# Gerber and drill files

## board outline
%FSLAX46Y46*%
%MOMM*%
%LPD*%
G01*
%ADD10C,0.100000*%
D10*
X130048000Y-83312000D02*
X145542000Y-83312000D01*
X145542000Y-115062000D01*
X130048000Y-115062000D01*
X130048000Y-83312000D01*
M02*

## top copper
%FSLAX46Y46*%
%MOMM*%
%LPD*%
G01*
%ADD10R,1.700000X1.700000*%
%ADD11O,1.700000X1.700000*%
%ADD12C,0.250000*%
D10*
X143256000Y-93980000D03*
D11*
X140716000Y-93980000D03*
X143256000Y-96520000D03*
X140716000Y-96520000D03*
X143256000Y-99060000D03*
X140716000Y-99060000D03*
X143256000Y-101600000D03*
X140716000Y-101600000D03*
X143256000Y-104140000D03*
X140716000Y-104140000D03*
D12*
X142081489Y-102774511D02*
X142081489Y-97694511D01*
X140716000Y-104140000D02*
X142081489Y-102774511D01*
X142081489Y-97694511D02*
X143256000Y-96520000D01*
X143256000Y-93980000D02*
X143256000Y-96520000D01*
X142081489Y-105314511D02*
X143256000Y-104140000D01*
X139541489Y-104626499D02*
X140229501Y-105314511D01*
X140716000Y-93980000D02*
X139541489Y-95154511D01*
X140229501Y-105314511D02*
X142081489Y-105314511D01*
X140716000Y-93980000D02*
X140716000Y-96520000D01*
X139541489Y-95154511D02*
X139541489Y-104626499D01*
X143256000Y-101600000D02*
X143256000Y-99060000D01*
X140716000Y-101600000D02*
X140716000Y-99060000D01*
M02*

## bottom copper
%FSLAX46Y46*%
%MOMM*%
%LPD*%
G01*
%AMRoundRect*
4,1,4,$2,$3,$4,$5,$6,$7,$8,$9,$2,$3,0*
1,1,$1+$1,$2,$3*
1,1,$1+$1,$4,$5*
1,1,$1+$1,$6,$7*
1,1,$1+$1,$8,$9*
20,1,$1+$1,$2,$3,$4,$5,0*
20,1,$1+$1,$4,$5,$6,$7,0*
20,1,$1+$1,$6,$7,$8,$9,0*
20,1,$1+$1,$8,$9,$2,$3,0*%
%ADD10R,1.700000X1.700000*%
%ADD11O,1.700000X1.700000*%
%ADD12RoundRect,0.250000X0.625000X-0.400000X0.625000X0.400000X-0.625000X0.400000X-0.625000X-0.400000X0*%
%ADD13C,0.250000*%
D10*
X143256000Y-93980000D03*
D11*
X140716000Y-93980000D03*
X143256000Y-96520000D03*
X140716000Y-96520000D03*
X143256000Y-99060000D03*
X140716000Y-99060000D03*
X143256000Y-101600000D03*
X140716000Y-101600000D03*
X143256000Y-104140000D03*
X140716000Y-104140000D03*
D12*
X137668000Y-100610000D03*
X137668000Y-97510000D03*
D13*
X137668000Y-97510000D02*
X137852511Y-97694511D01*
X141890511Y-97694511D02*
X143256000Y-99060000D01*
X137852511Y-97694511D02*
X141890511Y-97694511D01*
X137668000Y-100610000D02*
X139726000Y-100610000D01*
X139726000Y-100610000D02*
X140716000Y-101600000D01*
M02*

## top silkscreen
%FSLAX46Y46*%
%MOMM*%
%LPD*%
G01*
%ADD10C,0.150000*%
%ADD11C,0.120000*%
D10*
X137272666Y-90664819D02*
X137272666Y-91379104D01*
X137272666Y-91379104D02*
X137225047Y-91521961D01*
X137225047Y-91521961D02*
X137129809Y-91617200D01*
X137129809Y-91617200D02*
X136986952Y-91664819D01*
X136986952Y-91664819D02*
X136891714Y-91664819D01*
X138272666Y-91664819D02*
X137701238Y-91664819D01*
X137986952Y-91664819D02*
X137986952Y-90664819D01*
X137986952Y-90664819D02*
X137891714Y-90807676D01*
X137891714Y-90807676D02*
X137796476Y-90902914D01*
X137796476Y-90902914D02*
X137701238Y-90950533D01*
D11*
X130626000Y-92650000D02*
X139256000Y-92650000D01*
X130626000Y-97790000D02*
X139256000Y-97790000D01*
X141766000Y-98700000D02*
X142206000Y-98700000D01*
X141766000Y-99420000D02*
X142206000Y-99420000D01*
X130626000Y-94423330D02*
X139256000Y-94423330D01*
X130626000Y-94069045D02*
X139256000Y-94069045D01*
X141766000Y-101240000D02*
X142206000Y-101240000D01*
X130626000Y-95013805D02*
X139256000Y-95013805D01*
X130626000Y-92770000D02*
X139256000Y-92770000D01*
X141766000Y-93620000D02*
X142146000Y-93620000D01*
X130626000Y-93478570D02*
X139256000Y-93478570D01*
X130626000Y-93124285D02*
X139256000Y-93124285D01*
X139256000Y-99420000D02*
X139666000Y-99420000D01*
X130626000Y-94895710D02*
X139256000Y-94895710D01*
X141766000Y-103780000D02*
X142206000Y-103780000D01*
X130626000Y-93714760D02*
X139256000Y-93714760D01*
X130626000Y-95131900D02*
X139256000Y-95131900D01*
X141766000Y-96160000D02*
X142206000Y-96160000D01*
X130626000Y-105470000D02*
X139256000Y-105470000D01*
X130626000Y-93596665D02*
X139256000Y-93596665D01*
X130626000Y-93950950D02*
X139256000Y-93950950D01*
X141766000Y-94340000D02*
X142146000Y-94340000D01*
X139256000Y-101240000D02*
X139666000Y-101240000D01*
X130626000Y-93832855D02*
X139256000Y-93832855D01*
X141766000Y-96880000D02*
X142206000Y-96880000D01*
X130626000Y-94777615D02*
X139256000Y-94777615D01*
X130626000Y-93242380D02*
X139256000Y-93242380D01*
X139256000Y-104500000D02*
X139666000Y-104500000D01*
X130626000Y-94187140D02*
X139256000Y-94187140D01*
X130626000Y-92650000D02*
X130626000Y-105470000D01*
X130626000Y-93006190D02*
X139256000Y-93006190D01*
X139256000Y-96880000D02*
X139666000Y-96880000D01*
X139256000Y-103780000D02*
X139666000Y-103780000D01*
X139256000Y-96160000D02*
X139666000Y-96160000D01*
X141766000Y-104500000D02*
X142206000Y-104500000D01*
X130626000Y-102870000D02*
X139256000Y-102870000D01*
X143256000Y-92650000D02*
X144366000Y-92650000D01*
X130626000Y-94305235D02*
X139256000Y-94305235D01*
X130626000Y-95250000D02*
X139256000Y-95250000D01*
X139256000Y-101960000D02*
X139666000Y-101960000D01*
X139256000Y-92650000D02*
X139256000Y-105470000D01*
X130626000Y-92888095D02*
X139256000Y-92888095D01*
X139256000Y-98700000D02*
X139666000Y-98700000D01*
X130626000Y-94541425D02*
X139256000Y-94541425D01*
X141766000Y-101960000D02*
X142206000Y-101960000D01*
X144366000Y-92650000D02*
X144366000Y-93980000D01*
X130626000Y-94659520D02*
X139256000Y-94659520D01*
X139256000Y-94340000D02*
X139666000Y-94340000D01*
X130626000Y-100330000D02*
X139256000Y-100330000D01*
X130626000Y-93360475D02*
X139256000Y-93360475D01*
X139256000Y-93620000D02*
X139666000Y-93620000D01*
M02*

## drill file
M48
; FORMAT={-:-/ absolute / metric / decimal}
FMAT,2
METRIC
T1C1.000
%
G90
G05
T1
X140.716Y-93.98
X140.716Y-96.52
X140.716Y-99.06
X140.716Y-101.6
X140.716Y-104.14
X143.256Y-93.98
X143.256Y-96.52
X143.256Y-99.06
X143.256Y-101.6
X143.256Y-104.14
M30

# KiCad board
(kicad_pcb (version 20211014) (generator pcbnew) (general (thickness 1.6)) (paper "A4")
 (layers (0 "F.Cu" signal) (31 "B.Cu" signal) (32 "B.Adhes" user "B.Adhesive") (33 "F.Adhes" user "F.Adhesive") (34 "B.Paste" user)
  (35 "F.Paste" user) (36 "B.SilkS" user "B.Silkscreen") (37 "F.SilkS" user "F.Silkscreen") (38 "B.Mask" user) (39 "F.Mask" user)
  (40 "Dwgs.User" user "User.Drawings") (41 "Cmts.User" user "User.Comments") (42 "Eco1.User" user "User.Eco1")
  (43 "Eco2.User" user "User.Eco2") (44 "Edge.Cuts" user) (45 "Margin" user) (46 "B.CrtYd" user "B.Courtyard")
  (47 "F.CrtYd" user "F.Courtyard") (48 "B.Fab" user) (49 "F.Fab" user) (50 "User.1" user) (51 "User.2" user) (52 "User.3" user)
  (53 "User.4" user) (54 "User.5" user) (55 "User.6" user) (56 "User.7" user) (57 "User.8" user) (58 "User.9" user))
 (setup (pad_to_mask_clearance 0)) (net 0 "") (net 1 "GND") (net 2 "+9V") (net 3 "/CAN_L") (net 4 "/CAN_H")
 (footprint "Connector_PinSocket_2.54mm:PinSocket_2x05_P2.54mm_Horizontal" (layer "F.Cu") (at 143.256 93.98)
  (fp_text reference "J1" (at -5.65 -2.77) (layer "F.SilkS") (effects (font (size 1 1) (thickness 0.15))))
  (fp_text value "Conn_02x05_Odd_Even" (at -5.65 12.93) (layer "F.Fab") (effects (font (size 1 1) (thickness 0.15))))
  (fp_line (start -12.63 -1.33) (end -4 -1.33) (layer "F.SilkS") (width 0.12))
  (fp_line (start -12.63 3.81) (end -4 3.81) (layer "F.SilkS") (width 0.12))
  (fp_line (start -1.49 4.72) (end -1.05 4.72) (layer "F.SilkS") (width 0.12))
  (fp_line (start -1.49 5.44) (end -1.05 5.44) (layer "F.SilkS") (width 0.12))
  (fp_line (start -12.63 0.44333) (end -4 0.44333) (layer "F.SilkS") (width 0.12))
  (fp_line (start -12.63 0.089045) (end -4 0.089045) (layer "F.SilkS") (width 0.12))
  (fp_line (start -1.49 7.26) (end -1.05 7.26) (layer "F.SilkS") (width 0.12))
  (fp_line (start -12.63 1.033805) (end -4 1.033805) (layer "F.SilkS") (width 0.12))
  (fp_line (start -12.63 -1.21) (end -4 -1.21) (layer "F.SilkS") (width 0.12))
  (fp_line (start -1.49 -0.36) (end -1.11 -0.36) (layer "F.SilkS") (width 0.12))
  (fp_line (start -12.63 -0.50143) (end -4 -0.50143) (layer "F.SilkS") (width 0.12))
  (fp_line (start -12.63 -0.855715) (end -4 -0.855715) (layer "F.SilkS") (width 0.12))
  (fp_line (start -4 5.44) (end -3.59 5.44) (layer "F.SilkS") (width 0.12))
  (fp_line (start -12.63 0.91571) (end -4 0.91571) (layer "F.SilkS") (width 0.12))
  (fp_line (start -1.49 9.8) (end -1.05 9.8) (layer "F.SilkS") (width 0.12))
  (fp_line (start -12.63 -0.26524) (end -4 -0.26524) (layer "F.SilkS") (width 0.12))
  (fp_line (start -12.63 1.1519) (end -4 1.1519) (layer "F.SilkS") (width 0.12))
  (fp_line (start -1.49 2.18) (end -1.05 2.18) (layer "F.SilkS") (width 0.12))
  (fp_line (start -12.63 11.49) (end -4 11.49) (layer "F.SilkS") (width 0.12))
  (fp_line (start -12.63 -0.383335) (end -4 -0.383335) (layer "F.SilkS") (width 0.12))
  (fp_line (start -12.63 -0.02905) (end -4 -0.02905) (layer "F.SilkS") (width 0.12))
  (fp_line (start -1.49 0.36) (end -1.11 0.36) (layer "F.SilkS") (width 0.12))
  (fp_line (start -4 7.26) (end -3.59 7.26) (layer "F.SilkS") (width 0.12))
  (fp_line (start -12.63 -0.147145) (end -4 -0.147145) (layer "F.SilkS") (width 0.12))
  (fp_line (start -1.49 2.9) (end -1.05 2.9) (layer "F.SilkS") (width 0.12))
  (fp_line (start -12.63 0.797615) (end -4 0.797615) (layer "F.SilkS") (width 0.12))
  (fp_line (start -12.63 -0.73762) (end -4 -0.73762) (layer "F.SilkS") (width 0.12))
  (fp_line (start -4 10.52) (end -3.59 10.52) (layer "F.SilkS") (width 0.12))
  (fp_line (start -12.63 0.20714) (end -4 0.20714) (layer "F.SilkS") (width 0.12))
  (fp_line (start -12.63 -1.33) (end -12.63 11.49) (layer "F.SilkS") (width 0.12))
  (fp_line (start -12.63 -0.97381) (end -4 -0.97381) (layer "F.SilkS") (width 0.12))
  (fp_line (start -4 2.9) (end -3.59 2.9) (layer "F.SilkS") (width 0.12))
  (fp_line (start -4 9.8) (end -3.59 9.8) (layer "F.SilkS") (width 0.12))
  (fp_line (start -4 2.18) (end -3.59 2.18) (layer "F.SilkS") (width 0.12))
  (fp_line (start -1.49 10.52) (end -1.05 10.52) (layer "F.SilkS") (width 0.12))
  (fp_line (start -12.63 8.89) (end -4 8.89) (layer "F.SilkS") (width 0.12))
  (fp_line (start 0 -1.33) (end 1.11 -1.33) (layer "F.SilkS") (width 0.12))
  (fp_line (start -12.63 0.325235) (end -4 0.325235) (layer "F.SilkS") (width 0.12))
  (fp_line (start -12.63 1.27) (end -4 1.27) (layer "F.SilkS") (width 0.12))
  (fp_line (start -4 7.98) (end -3.59 7.98) (layer "F.SilkS") (width 0.12))
  (fp_line (start -4 -1.33) (end -4 11.49) (layer "F.SilkS") (width 0.12))
  (fp_line (start -12.63 -1.091905) (end -4 -1.091905) (layer "F.SilkS") (width 0.12))
  (fp_line (start -4 4.72) (end -3.59 4.72) (layer "F.SilkS") (width 0.12))
  (fp_line (start -12.63 0.561425) (end -4 0.561425) (layer "F.SilkS") (width 0.12))
  (fp_line (start -1.49 7.98) (end -1.05 7.98) (layer "F.SilkS") (width 0.12))
  (fp_line (start 1.11 -1.33) (end 1.11 0) (layer "F.SilkS") (width 0.12))
  (fp_line (start -12.63 0.67952) (end -4 0.67952) (layer "F.SilkS") (width 0.12))
  (fp_line (start -4 0.36) (end -3.59 0.36) (layer "F.SilkS") (width 0.12))
  (fp_line (start -12.63 6.35) (end -4 6.35) (layer "F.SilkS") (width 0.12))
  (fp_line (start -12.63 -0.619525) (end -4 -0.619525) (layer "F.SilkS") (width 0.12))
  (fp_line (start -4 -0.36) (end -3.59 -0.36) (layer "F.SilkS") (width 0.12))
  (pad "1" thru_hole rect (at 0 0) (size 1.7 1.7) (drill 1) (layers *.Cu *.Mask) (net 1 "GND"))
  (pad "2" thru_hole oval (at -2.54 0) (size 1.7 1.7) (drill 1) (layers *.Cu *.Mask) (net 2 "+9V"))
  (pad "3" thru_hole oval (at 0 2.54) (size 1.7 1.7) (drill 1) (layers *.Cu *.Mask) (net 1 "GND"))
  (pad "4" thru_hole oval (at -2.54 2.54) (size 1.7 1.7) (drill 1) (layers *.Cu *.Mask) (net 2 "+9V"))
  (pad "5" thru_hole oval (at 0 5.08) (size 1.7 1.7) (drill 1) (layers *.Cu *.Mask) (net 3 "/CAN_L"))
  (pad "6" thru_hole oval (at -2.54 5.08) (size 1.7 1.7) (drill 1) (layers *.Cu *.Mask) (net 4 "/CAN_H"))
  (pad "7" thru_hole oval (at 0 7.62) (size 1.7 1.7) (drill 1) (layers *.Cu *.Mask) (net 3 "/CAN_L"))
  (pad "8" thru_hole oval (at -2.54 7.62) (size 1.7 1.7) (drill 1) (layers *.Cu *.Mask) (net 4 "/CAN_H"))
  (pad "9" thru_hole oval (at 0 10.16) (size 1.7 1.7) (drill 1) (layers *.Cu *.Mask) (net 2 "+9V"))
  (pad "10" thru_hole oval (at -2.54 10.16) (size 1.7 1.7) (drill 1) (layers *.Cu *.Mask) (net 1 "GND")))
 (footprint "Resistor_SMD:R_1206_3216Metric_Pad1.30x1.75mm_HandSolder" (layer "B.Cu") (at 137.668 99.06 90)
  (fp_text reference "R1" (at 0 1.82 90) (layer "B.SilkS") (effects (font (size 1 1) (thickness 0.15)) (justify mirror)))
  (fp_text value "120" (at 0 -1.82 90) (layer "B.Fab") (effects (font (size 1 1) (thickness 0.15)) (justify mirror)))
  (pad "1" smd roundrect (at -1.55 0 90) (size 1.3 1.75) (layers "B.Cu" "B.Paste" "B.Mask") (roundrect_rratio 0.1923076923) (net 4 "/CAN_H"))
  (pad "2" smd roundrect (at 1.55 0 90) (size 1.3 1.75) (layers "B.Cu" "B.Paste" "B.Mask") (roundrect_rratio 0.1923076923) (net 3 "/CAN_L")))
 (gr_rect (start 130.048 83.312) (end 145.542 115.062) (layer "Edge.Cuts") (width 0.1) (fill none))
 (segment (start 142.081489 102.774511) (end 142.081489 97.694511) (width 0.25) (layer "F.Cu") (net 1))
 (segment (start 140.716 104.14) (end 142.081489 102.774511) (width 0.25) (layer "F.Cu") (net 1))
 (segment (start 142.081489 97.694511) (end 143.256 96.52) (width 0.25) (layer "F.Cu") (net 1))
 (segment (start 143.256 93.98) (end 143.256 96.52) (width 0.25) (layer "F.Cu") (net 1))
 (segment (start 142.081489 105.314511) (end 143.256 104.14) (width 0.25) (layer "F.Cu") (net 2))
 (segment (start 139.541489 104.626499) (end 140.229501 105.314511) (width 0.25) (layer "F.Cu") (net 2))
 (segment (start 140.716 93.98) (end 139.541489 95.154511) (width 0.25) (layer "F.Cu") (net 2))
 (segment (start 140.229501 105.314511) (end 142.081489 105.314511) (width 0.25) (layer "F.Cu") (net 2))
 (segment (start 140.716 93.98) (end 140.716 96.52) (width 0.25) (layer "F.Cu") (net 2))
 (segment (start 139.541489 95.154511) (end 139.541489 104.626499) (width 0.25) (layer "F.Cu") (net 2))
 (segment (start 143.256 101.6) (end 143.256 99.06) (width 0.25) (layer "F.Cu") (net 3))
 (segment (start 137.668 97.51) (end 137.852511 97.694511) (width 0.25) (layer "B.Cu") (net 3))
 (segment (start 141.890511 97.694511) (end 143.256 99.06) (width 0.25) (layer "B.Cu") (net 3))
 (segment (start 137.852511 97.694511) (end 141.890511 97.694511) (width 0.25) (layer "B.Cu") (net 3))
 (segment (start 140.716 101.6) (end 140.716 99.06) (width 0.25) (layer "F.Cu") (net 4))
 (segment (start 137.668 100.61) (end 139.726 100.61) (width 0.25) (layer "B.Cu") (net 4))
 (segment (start 139.726 100.61) (end 140.716 101.6) (width 0.25) (layer "B.Cu") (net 4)))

